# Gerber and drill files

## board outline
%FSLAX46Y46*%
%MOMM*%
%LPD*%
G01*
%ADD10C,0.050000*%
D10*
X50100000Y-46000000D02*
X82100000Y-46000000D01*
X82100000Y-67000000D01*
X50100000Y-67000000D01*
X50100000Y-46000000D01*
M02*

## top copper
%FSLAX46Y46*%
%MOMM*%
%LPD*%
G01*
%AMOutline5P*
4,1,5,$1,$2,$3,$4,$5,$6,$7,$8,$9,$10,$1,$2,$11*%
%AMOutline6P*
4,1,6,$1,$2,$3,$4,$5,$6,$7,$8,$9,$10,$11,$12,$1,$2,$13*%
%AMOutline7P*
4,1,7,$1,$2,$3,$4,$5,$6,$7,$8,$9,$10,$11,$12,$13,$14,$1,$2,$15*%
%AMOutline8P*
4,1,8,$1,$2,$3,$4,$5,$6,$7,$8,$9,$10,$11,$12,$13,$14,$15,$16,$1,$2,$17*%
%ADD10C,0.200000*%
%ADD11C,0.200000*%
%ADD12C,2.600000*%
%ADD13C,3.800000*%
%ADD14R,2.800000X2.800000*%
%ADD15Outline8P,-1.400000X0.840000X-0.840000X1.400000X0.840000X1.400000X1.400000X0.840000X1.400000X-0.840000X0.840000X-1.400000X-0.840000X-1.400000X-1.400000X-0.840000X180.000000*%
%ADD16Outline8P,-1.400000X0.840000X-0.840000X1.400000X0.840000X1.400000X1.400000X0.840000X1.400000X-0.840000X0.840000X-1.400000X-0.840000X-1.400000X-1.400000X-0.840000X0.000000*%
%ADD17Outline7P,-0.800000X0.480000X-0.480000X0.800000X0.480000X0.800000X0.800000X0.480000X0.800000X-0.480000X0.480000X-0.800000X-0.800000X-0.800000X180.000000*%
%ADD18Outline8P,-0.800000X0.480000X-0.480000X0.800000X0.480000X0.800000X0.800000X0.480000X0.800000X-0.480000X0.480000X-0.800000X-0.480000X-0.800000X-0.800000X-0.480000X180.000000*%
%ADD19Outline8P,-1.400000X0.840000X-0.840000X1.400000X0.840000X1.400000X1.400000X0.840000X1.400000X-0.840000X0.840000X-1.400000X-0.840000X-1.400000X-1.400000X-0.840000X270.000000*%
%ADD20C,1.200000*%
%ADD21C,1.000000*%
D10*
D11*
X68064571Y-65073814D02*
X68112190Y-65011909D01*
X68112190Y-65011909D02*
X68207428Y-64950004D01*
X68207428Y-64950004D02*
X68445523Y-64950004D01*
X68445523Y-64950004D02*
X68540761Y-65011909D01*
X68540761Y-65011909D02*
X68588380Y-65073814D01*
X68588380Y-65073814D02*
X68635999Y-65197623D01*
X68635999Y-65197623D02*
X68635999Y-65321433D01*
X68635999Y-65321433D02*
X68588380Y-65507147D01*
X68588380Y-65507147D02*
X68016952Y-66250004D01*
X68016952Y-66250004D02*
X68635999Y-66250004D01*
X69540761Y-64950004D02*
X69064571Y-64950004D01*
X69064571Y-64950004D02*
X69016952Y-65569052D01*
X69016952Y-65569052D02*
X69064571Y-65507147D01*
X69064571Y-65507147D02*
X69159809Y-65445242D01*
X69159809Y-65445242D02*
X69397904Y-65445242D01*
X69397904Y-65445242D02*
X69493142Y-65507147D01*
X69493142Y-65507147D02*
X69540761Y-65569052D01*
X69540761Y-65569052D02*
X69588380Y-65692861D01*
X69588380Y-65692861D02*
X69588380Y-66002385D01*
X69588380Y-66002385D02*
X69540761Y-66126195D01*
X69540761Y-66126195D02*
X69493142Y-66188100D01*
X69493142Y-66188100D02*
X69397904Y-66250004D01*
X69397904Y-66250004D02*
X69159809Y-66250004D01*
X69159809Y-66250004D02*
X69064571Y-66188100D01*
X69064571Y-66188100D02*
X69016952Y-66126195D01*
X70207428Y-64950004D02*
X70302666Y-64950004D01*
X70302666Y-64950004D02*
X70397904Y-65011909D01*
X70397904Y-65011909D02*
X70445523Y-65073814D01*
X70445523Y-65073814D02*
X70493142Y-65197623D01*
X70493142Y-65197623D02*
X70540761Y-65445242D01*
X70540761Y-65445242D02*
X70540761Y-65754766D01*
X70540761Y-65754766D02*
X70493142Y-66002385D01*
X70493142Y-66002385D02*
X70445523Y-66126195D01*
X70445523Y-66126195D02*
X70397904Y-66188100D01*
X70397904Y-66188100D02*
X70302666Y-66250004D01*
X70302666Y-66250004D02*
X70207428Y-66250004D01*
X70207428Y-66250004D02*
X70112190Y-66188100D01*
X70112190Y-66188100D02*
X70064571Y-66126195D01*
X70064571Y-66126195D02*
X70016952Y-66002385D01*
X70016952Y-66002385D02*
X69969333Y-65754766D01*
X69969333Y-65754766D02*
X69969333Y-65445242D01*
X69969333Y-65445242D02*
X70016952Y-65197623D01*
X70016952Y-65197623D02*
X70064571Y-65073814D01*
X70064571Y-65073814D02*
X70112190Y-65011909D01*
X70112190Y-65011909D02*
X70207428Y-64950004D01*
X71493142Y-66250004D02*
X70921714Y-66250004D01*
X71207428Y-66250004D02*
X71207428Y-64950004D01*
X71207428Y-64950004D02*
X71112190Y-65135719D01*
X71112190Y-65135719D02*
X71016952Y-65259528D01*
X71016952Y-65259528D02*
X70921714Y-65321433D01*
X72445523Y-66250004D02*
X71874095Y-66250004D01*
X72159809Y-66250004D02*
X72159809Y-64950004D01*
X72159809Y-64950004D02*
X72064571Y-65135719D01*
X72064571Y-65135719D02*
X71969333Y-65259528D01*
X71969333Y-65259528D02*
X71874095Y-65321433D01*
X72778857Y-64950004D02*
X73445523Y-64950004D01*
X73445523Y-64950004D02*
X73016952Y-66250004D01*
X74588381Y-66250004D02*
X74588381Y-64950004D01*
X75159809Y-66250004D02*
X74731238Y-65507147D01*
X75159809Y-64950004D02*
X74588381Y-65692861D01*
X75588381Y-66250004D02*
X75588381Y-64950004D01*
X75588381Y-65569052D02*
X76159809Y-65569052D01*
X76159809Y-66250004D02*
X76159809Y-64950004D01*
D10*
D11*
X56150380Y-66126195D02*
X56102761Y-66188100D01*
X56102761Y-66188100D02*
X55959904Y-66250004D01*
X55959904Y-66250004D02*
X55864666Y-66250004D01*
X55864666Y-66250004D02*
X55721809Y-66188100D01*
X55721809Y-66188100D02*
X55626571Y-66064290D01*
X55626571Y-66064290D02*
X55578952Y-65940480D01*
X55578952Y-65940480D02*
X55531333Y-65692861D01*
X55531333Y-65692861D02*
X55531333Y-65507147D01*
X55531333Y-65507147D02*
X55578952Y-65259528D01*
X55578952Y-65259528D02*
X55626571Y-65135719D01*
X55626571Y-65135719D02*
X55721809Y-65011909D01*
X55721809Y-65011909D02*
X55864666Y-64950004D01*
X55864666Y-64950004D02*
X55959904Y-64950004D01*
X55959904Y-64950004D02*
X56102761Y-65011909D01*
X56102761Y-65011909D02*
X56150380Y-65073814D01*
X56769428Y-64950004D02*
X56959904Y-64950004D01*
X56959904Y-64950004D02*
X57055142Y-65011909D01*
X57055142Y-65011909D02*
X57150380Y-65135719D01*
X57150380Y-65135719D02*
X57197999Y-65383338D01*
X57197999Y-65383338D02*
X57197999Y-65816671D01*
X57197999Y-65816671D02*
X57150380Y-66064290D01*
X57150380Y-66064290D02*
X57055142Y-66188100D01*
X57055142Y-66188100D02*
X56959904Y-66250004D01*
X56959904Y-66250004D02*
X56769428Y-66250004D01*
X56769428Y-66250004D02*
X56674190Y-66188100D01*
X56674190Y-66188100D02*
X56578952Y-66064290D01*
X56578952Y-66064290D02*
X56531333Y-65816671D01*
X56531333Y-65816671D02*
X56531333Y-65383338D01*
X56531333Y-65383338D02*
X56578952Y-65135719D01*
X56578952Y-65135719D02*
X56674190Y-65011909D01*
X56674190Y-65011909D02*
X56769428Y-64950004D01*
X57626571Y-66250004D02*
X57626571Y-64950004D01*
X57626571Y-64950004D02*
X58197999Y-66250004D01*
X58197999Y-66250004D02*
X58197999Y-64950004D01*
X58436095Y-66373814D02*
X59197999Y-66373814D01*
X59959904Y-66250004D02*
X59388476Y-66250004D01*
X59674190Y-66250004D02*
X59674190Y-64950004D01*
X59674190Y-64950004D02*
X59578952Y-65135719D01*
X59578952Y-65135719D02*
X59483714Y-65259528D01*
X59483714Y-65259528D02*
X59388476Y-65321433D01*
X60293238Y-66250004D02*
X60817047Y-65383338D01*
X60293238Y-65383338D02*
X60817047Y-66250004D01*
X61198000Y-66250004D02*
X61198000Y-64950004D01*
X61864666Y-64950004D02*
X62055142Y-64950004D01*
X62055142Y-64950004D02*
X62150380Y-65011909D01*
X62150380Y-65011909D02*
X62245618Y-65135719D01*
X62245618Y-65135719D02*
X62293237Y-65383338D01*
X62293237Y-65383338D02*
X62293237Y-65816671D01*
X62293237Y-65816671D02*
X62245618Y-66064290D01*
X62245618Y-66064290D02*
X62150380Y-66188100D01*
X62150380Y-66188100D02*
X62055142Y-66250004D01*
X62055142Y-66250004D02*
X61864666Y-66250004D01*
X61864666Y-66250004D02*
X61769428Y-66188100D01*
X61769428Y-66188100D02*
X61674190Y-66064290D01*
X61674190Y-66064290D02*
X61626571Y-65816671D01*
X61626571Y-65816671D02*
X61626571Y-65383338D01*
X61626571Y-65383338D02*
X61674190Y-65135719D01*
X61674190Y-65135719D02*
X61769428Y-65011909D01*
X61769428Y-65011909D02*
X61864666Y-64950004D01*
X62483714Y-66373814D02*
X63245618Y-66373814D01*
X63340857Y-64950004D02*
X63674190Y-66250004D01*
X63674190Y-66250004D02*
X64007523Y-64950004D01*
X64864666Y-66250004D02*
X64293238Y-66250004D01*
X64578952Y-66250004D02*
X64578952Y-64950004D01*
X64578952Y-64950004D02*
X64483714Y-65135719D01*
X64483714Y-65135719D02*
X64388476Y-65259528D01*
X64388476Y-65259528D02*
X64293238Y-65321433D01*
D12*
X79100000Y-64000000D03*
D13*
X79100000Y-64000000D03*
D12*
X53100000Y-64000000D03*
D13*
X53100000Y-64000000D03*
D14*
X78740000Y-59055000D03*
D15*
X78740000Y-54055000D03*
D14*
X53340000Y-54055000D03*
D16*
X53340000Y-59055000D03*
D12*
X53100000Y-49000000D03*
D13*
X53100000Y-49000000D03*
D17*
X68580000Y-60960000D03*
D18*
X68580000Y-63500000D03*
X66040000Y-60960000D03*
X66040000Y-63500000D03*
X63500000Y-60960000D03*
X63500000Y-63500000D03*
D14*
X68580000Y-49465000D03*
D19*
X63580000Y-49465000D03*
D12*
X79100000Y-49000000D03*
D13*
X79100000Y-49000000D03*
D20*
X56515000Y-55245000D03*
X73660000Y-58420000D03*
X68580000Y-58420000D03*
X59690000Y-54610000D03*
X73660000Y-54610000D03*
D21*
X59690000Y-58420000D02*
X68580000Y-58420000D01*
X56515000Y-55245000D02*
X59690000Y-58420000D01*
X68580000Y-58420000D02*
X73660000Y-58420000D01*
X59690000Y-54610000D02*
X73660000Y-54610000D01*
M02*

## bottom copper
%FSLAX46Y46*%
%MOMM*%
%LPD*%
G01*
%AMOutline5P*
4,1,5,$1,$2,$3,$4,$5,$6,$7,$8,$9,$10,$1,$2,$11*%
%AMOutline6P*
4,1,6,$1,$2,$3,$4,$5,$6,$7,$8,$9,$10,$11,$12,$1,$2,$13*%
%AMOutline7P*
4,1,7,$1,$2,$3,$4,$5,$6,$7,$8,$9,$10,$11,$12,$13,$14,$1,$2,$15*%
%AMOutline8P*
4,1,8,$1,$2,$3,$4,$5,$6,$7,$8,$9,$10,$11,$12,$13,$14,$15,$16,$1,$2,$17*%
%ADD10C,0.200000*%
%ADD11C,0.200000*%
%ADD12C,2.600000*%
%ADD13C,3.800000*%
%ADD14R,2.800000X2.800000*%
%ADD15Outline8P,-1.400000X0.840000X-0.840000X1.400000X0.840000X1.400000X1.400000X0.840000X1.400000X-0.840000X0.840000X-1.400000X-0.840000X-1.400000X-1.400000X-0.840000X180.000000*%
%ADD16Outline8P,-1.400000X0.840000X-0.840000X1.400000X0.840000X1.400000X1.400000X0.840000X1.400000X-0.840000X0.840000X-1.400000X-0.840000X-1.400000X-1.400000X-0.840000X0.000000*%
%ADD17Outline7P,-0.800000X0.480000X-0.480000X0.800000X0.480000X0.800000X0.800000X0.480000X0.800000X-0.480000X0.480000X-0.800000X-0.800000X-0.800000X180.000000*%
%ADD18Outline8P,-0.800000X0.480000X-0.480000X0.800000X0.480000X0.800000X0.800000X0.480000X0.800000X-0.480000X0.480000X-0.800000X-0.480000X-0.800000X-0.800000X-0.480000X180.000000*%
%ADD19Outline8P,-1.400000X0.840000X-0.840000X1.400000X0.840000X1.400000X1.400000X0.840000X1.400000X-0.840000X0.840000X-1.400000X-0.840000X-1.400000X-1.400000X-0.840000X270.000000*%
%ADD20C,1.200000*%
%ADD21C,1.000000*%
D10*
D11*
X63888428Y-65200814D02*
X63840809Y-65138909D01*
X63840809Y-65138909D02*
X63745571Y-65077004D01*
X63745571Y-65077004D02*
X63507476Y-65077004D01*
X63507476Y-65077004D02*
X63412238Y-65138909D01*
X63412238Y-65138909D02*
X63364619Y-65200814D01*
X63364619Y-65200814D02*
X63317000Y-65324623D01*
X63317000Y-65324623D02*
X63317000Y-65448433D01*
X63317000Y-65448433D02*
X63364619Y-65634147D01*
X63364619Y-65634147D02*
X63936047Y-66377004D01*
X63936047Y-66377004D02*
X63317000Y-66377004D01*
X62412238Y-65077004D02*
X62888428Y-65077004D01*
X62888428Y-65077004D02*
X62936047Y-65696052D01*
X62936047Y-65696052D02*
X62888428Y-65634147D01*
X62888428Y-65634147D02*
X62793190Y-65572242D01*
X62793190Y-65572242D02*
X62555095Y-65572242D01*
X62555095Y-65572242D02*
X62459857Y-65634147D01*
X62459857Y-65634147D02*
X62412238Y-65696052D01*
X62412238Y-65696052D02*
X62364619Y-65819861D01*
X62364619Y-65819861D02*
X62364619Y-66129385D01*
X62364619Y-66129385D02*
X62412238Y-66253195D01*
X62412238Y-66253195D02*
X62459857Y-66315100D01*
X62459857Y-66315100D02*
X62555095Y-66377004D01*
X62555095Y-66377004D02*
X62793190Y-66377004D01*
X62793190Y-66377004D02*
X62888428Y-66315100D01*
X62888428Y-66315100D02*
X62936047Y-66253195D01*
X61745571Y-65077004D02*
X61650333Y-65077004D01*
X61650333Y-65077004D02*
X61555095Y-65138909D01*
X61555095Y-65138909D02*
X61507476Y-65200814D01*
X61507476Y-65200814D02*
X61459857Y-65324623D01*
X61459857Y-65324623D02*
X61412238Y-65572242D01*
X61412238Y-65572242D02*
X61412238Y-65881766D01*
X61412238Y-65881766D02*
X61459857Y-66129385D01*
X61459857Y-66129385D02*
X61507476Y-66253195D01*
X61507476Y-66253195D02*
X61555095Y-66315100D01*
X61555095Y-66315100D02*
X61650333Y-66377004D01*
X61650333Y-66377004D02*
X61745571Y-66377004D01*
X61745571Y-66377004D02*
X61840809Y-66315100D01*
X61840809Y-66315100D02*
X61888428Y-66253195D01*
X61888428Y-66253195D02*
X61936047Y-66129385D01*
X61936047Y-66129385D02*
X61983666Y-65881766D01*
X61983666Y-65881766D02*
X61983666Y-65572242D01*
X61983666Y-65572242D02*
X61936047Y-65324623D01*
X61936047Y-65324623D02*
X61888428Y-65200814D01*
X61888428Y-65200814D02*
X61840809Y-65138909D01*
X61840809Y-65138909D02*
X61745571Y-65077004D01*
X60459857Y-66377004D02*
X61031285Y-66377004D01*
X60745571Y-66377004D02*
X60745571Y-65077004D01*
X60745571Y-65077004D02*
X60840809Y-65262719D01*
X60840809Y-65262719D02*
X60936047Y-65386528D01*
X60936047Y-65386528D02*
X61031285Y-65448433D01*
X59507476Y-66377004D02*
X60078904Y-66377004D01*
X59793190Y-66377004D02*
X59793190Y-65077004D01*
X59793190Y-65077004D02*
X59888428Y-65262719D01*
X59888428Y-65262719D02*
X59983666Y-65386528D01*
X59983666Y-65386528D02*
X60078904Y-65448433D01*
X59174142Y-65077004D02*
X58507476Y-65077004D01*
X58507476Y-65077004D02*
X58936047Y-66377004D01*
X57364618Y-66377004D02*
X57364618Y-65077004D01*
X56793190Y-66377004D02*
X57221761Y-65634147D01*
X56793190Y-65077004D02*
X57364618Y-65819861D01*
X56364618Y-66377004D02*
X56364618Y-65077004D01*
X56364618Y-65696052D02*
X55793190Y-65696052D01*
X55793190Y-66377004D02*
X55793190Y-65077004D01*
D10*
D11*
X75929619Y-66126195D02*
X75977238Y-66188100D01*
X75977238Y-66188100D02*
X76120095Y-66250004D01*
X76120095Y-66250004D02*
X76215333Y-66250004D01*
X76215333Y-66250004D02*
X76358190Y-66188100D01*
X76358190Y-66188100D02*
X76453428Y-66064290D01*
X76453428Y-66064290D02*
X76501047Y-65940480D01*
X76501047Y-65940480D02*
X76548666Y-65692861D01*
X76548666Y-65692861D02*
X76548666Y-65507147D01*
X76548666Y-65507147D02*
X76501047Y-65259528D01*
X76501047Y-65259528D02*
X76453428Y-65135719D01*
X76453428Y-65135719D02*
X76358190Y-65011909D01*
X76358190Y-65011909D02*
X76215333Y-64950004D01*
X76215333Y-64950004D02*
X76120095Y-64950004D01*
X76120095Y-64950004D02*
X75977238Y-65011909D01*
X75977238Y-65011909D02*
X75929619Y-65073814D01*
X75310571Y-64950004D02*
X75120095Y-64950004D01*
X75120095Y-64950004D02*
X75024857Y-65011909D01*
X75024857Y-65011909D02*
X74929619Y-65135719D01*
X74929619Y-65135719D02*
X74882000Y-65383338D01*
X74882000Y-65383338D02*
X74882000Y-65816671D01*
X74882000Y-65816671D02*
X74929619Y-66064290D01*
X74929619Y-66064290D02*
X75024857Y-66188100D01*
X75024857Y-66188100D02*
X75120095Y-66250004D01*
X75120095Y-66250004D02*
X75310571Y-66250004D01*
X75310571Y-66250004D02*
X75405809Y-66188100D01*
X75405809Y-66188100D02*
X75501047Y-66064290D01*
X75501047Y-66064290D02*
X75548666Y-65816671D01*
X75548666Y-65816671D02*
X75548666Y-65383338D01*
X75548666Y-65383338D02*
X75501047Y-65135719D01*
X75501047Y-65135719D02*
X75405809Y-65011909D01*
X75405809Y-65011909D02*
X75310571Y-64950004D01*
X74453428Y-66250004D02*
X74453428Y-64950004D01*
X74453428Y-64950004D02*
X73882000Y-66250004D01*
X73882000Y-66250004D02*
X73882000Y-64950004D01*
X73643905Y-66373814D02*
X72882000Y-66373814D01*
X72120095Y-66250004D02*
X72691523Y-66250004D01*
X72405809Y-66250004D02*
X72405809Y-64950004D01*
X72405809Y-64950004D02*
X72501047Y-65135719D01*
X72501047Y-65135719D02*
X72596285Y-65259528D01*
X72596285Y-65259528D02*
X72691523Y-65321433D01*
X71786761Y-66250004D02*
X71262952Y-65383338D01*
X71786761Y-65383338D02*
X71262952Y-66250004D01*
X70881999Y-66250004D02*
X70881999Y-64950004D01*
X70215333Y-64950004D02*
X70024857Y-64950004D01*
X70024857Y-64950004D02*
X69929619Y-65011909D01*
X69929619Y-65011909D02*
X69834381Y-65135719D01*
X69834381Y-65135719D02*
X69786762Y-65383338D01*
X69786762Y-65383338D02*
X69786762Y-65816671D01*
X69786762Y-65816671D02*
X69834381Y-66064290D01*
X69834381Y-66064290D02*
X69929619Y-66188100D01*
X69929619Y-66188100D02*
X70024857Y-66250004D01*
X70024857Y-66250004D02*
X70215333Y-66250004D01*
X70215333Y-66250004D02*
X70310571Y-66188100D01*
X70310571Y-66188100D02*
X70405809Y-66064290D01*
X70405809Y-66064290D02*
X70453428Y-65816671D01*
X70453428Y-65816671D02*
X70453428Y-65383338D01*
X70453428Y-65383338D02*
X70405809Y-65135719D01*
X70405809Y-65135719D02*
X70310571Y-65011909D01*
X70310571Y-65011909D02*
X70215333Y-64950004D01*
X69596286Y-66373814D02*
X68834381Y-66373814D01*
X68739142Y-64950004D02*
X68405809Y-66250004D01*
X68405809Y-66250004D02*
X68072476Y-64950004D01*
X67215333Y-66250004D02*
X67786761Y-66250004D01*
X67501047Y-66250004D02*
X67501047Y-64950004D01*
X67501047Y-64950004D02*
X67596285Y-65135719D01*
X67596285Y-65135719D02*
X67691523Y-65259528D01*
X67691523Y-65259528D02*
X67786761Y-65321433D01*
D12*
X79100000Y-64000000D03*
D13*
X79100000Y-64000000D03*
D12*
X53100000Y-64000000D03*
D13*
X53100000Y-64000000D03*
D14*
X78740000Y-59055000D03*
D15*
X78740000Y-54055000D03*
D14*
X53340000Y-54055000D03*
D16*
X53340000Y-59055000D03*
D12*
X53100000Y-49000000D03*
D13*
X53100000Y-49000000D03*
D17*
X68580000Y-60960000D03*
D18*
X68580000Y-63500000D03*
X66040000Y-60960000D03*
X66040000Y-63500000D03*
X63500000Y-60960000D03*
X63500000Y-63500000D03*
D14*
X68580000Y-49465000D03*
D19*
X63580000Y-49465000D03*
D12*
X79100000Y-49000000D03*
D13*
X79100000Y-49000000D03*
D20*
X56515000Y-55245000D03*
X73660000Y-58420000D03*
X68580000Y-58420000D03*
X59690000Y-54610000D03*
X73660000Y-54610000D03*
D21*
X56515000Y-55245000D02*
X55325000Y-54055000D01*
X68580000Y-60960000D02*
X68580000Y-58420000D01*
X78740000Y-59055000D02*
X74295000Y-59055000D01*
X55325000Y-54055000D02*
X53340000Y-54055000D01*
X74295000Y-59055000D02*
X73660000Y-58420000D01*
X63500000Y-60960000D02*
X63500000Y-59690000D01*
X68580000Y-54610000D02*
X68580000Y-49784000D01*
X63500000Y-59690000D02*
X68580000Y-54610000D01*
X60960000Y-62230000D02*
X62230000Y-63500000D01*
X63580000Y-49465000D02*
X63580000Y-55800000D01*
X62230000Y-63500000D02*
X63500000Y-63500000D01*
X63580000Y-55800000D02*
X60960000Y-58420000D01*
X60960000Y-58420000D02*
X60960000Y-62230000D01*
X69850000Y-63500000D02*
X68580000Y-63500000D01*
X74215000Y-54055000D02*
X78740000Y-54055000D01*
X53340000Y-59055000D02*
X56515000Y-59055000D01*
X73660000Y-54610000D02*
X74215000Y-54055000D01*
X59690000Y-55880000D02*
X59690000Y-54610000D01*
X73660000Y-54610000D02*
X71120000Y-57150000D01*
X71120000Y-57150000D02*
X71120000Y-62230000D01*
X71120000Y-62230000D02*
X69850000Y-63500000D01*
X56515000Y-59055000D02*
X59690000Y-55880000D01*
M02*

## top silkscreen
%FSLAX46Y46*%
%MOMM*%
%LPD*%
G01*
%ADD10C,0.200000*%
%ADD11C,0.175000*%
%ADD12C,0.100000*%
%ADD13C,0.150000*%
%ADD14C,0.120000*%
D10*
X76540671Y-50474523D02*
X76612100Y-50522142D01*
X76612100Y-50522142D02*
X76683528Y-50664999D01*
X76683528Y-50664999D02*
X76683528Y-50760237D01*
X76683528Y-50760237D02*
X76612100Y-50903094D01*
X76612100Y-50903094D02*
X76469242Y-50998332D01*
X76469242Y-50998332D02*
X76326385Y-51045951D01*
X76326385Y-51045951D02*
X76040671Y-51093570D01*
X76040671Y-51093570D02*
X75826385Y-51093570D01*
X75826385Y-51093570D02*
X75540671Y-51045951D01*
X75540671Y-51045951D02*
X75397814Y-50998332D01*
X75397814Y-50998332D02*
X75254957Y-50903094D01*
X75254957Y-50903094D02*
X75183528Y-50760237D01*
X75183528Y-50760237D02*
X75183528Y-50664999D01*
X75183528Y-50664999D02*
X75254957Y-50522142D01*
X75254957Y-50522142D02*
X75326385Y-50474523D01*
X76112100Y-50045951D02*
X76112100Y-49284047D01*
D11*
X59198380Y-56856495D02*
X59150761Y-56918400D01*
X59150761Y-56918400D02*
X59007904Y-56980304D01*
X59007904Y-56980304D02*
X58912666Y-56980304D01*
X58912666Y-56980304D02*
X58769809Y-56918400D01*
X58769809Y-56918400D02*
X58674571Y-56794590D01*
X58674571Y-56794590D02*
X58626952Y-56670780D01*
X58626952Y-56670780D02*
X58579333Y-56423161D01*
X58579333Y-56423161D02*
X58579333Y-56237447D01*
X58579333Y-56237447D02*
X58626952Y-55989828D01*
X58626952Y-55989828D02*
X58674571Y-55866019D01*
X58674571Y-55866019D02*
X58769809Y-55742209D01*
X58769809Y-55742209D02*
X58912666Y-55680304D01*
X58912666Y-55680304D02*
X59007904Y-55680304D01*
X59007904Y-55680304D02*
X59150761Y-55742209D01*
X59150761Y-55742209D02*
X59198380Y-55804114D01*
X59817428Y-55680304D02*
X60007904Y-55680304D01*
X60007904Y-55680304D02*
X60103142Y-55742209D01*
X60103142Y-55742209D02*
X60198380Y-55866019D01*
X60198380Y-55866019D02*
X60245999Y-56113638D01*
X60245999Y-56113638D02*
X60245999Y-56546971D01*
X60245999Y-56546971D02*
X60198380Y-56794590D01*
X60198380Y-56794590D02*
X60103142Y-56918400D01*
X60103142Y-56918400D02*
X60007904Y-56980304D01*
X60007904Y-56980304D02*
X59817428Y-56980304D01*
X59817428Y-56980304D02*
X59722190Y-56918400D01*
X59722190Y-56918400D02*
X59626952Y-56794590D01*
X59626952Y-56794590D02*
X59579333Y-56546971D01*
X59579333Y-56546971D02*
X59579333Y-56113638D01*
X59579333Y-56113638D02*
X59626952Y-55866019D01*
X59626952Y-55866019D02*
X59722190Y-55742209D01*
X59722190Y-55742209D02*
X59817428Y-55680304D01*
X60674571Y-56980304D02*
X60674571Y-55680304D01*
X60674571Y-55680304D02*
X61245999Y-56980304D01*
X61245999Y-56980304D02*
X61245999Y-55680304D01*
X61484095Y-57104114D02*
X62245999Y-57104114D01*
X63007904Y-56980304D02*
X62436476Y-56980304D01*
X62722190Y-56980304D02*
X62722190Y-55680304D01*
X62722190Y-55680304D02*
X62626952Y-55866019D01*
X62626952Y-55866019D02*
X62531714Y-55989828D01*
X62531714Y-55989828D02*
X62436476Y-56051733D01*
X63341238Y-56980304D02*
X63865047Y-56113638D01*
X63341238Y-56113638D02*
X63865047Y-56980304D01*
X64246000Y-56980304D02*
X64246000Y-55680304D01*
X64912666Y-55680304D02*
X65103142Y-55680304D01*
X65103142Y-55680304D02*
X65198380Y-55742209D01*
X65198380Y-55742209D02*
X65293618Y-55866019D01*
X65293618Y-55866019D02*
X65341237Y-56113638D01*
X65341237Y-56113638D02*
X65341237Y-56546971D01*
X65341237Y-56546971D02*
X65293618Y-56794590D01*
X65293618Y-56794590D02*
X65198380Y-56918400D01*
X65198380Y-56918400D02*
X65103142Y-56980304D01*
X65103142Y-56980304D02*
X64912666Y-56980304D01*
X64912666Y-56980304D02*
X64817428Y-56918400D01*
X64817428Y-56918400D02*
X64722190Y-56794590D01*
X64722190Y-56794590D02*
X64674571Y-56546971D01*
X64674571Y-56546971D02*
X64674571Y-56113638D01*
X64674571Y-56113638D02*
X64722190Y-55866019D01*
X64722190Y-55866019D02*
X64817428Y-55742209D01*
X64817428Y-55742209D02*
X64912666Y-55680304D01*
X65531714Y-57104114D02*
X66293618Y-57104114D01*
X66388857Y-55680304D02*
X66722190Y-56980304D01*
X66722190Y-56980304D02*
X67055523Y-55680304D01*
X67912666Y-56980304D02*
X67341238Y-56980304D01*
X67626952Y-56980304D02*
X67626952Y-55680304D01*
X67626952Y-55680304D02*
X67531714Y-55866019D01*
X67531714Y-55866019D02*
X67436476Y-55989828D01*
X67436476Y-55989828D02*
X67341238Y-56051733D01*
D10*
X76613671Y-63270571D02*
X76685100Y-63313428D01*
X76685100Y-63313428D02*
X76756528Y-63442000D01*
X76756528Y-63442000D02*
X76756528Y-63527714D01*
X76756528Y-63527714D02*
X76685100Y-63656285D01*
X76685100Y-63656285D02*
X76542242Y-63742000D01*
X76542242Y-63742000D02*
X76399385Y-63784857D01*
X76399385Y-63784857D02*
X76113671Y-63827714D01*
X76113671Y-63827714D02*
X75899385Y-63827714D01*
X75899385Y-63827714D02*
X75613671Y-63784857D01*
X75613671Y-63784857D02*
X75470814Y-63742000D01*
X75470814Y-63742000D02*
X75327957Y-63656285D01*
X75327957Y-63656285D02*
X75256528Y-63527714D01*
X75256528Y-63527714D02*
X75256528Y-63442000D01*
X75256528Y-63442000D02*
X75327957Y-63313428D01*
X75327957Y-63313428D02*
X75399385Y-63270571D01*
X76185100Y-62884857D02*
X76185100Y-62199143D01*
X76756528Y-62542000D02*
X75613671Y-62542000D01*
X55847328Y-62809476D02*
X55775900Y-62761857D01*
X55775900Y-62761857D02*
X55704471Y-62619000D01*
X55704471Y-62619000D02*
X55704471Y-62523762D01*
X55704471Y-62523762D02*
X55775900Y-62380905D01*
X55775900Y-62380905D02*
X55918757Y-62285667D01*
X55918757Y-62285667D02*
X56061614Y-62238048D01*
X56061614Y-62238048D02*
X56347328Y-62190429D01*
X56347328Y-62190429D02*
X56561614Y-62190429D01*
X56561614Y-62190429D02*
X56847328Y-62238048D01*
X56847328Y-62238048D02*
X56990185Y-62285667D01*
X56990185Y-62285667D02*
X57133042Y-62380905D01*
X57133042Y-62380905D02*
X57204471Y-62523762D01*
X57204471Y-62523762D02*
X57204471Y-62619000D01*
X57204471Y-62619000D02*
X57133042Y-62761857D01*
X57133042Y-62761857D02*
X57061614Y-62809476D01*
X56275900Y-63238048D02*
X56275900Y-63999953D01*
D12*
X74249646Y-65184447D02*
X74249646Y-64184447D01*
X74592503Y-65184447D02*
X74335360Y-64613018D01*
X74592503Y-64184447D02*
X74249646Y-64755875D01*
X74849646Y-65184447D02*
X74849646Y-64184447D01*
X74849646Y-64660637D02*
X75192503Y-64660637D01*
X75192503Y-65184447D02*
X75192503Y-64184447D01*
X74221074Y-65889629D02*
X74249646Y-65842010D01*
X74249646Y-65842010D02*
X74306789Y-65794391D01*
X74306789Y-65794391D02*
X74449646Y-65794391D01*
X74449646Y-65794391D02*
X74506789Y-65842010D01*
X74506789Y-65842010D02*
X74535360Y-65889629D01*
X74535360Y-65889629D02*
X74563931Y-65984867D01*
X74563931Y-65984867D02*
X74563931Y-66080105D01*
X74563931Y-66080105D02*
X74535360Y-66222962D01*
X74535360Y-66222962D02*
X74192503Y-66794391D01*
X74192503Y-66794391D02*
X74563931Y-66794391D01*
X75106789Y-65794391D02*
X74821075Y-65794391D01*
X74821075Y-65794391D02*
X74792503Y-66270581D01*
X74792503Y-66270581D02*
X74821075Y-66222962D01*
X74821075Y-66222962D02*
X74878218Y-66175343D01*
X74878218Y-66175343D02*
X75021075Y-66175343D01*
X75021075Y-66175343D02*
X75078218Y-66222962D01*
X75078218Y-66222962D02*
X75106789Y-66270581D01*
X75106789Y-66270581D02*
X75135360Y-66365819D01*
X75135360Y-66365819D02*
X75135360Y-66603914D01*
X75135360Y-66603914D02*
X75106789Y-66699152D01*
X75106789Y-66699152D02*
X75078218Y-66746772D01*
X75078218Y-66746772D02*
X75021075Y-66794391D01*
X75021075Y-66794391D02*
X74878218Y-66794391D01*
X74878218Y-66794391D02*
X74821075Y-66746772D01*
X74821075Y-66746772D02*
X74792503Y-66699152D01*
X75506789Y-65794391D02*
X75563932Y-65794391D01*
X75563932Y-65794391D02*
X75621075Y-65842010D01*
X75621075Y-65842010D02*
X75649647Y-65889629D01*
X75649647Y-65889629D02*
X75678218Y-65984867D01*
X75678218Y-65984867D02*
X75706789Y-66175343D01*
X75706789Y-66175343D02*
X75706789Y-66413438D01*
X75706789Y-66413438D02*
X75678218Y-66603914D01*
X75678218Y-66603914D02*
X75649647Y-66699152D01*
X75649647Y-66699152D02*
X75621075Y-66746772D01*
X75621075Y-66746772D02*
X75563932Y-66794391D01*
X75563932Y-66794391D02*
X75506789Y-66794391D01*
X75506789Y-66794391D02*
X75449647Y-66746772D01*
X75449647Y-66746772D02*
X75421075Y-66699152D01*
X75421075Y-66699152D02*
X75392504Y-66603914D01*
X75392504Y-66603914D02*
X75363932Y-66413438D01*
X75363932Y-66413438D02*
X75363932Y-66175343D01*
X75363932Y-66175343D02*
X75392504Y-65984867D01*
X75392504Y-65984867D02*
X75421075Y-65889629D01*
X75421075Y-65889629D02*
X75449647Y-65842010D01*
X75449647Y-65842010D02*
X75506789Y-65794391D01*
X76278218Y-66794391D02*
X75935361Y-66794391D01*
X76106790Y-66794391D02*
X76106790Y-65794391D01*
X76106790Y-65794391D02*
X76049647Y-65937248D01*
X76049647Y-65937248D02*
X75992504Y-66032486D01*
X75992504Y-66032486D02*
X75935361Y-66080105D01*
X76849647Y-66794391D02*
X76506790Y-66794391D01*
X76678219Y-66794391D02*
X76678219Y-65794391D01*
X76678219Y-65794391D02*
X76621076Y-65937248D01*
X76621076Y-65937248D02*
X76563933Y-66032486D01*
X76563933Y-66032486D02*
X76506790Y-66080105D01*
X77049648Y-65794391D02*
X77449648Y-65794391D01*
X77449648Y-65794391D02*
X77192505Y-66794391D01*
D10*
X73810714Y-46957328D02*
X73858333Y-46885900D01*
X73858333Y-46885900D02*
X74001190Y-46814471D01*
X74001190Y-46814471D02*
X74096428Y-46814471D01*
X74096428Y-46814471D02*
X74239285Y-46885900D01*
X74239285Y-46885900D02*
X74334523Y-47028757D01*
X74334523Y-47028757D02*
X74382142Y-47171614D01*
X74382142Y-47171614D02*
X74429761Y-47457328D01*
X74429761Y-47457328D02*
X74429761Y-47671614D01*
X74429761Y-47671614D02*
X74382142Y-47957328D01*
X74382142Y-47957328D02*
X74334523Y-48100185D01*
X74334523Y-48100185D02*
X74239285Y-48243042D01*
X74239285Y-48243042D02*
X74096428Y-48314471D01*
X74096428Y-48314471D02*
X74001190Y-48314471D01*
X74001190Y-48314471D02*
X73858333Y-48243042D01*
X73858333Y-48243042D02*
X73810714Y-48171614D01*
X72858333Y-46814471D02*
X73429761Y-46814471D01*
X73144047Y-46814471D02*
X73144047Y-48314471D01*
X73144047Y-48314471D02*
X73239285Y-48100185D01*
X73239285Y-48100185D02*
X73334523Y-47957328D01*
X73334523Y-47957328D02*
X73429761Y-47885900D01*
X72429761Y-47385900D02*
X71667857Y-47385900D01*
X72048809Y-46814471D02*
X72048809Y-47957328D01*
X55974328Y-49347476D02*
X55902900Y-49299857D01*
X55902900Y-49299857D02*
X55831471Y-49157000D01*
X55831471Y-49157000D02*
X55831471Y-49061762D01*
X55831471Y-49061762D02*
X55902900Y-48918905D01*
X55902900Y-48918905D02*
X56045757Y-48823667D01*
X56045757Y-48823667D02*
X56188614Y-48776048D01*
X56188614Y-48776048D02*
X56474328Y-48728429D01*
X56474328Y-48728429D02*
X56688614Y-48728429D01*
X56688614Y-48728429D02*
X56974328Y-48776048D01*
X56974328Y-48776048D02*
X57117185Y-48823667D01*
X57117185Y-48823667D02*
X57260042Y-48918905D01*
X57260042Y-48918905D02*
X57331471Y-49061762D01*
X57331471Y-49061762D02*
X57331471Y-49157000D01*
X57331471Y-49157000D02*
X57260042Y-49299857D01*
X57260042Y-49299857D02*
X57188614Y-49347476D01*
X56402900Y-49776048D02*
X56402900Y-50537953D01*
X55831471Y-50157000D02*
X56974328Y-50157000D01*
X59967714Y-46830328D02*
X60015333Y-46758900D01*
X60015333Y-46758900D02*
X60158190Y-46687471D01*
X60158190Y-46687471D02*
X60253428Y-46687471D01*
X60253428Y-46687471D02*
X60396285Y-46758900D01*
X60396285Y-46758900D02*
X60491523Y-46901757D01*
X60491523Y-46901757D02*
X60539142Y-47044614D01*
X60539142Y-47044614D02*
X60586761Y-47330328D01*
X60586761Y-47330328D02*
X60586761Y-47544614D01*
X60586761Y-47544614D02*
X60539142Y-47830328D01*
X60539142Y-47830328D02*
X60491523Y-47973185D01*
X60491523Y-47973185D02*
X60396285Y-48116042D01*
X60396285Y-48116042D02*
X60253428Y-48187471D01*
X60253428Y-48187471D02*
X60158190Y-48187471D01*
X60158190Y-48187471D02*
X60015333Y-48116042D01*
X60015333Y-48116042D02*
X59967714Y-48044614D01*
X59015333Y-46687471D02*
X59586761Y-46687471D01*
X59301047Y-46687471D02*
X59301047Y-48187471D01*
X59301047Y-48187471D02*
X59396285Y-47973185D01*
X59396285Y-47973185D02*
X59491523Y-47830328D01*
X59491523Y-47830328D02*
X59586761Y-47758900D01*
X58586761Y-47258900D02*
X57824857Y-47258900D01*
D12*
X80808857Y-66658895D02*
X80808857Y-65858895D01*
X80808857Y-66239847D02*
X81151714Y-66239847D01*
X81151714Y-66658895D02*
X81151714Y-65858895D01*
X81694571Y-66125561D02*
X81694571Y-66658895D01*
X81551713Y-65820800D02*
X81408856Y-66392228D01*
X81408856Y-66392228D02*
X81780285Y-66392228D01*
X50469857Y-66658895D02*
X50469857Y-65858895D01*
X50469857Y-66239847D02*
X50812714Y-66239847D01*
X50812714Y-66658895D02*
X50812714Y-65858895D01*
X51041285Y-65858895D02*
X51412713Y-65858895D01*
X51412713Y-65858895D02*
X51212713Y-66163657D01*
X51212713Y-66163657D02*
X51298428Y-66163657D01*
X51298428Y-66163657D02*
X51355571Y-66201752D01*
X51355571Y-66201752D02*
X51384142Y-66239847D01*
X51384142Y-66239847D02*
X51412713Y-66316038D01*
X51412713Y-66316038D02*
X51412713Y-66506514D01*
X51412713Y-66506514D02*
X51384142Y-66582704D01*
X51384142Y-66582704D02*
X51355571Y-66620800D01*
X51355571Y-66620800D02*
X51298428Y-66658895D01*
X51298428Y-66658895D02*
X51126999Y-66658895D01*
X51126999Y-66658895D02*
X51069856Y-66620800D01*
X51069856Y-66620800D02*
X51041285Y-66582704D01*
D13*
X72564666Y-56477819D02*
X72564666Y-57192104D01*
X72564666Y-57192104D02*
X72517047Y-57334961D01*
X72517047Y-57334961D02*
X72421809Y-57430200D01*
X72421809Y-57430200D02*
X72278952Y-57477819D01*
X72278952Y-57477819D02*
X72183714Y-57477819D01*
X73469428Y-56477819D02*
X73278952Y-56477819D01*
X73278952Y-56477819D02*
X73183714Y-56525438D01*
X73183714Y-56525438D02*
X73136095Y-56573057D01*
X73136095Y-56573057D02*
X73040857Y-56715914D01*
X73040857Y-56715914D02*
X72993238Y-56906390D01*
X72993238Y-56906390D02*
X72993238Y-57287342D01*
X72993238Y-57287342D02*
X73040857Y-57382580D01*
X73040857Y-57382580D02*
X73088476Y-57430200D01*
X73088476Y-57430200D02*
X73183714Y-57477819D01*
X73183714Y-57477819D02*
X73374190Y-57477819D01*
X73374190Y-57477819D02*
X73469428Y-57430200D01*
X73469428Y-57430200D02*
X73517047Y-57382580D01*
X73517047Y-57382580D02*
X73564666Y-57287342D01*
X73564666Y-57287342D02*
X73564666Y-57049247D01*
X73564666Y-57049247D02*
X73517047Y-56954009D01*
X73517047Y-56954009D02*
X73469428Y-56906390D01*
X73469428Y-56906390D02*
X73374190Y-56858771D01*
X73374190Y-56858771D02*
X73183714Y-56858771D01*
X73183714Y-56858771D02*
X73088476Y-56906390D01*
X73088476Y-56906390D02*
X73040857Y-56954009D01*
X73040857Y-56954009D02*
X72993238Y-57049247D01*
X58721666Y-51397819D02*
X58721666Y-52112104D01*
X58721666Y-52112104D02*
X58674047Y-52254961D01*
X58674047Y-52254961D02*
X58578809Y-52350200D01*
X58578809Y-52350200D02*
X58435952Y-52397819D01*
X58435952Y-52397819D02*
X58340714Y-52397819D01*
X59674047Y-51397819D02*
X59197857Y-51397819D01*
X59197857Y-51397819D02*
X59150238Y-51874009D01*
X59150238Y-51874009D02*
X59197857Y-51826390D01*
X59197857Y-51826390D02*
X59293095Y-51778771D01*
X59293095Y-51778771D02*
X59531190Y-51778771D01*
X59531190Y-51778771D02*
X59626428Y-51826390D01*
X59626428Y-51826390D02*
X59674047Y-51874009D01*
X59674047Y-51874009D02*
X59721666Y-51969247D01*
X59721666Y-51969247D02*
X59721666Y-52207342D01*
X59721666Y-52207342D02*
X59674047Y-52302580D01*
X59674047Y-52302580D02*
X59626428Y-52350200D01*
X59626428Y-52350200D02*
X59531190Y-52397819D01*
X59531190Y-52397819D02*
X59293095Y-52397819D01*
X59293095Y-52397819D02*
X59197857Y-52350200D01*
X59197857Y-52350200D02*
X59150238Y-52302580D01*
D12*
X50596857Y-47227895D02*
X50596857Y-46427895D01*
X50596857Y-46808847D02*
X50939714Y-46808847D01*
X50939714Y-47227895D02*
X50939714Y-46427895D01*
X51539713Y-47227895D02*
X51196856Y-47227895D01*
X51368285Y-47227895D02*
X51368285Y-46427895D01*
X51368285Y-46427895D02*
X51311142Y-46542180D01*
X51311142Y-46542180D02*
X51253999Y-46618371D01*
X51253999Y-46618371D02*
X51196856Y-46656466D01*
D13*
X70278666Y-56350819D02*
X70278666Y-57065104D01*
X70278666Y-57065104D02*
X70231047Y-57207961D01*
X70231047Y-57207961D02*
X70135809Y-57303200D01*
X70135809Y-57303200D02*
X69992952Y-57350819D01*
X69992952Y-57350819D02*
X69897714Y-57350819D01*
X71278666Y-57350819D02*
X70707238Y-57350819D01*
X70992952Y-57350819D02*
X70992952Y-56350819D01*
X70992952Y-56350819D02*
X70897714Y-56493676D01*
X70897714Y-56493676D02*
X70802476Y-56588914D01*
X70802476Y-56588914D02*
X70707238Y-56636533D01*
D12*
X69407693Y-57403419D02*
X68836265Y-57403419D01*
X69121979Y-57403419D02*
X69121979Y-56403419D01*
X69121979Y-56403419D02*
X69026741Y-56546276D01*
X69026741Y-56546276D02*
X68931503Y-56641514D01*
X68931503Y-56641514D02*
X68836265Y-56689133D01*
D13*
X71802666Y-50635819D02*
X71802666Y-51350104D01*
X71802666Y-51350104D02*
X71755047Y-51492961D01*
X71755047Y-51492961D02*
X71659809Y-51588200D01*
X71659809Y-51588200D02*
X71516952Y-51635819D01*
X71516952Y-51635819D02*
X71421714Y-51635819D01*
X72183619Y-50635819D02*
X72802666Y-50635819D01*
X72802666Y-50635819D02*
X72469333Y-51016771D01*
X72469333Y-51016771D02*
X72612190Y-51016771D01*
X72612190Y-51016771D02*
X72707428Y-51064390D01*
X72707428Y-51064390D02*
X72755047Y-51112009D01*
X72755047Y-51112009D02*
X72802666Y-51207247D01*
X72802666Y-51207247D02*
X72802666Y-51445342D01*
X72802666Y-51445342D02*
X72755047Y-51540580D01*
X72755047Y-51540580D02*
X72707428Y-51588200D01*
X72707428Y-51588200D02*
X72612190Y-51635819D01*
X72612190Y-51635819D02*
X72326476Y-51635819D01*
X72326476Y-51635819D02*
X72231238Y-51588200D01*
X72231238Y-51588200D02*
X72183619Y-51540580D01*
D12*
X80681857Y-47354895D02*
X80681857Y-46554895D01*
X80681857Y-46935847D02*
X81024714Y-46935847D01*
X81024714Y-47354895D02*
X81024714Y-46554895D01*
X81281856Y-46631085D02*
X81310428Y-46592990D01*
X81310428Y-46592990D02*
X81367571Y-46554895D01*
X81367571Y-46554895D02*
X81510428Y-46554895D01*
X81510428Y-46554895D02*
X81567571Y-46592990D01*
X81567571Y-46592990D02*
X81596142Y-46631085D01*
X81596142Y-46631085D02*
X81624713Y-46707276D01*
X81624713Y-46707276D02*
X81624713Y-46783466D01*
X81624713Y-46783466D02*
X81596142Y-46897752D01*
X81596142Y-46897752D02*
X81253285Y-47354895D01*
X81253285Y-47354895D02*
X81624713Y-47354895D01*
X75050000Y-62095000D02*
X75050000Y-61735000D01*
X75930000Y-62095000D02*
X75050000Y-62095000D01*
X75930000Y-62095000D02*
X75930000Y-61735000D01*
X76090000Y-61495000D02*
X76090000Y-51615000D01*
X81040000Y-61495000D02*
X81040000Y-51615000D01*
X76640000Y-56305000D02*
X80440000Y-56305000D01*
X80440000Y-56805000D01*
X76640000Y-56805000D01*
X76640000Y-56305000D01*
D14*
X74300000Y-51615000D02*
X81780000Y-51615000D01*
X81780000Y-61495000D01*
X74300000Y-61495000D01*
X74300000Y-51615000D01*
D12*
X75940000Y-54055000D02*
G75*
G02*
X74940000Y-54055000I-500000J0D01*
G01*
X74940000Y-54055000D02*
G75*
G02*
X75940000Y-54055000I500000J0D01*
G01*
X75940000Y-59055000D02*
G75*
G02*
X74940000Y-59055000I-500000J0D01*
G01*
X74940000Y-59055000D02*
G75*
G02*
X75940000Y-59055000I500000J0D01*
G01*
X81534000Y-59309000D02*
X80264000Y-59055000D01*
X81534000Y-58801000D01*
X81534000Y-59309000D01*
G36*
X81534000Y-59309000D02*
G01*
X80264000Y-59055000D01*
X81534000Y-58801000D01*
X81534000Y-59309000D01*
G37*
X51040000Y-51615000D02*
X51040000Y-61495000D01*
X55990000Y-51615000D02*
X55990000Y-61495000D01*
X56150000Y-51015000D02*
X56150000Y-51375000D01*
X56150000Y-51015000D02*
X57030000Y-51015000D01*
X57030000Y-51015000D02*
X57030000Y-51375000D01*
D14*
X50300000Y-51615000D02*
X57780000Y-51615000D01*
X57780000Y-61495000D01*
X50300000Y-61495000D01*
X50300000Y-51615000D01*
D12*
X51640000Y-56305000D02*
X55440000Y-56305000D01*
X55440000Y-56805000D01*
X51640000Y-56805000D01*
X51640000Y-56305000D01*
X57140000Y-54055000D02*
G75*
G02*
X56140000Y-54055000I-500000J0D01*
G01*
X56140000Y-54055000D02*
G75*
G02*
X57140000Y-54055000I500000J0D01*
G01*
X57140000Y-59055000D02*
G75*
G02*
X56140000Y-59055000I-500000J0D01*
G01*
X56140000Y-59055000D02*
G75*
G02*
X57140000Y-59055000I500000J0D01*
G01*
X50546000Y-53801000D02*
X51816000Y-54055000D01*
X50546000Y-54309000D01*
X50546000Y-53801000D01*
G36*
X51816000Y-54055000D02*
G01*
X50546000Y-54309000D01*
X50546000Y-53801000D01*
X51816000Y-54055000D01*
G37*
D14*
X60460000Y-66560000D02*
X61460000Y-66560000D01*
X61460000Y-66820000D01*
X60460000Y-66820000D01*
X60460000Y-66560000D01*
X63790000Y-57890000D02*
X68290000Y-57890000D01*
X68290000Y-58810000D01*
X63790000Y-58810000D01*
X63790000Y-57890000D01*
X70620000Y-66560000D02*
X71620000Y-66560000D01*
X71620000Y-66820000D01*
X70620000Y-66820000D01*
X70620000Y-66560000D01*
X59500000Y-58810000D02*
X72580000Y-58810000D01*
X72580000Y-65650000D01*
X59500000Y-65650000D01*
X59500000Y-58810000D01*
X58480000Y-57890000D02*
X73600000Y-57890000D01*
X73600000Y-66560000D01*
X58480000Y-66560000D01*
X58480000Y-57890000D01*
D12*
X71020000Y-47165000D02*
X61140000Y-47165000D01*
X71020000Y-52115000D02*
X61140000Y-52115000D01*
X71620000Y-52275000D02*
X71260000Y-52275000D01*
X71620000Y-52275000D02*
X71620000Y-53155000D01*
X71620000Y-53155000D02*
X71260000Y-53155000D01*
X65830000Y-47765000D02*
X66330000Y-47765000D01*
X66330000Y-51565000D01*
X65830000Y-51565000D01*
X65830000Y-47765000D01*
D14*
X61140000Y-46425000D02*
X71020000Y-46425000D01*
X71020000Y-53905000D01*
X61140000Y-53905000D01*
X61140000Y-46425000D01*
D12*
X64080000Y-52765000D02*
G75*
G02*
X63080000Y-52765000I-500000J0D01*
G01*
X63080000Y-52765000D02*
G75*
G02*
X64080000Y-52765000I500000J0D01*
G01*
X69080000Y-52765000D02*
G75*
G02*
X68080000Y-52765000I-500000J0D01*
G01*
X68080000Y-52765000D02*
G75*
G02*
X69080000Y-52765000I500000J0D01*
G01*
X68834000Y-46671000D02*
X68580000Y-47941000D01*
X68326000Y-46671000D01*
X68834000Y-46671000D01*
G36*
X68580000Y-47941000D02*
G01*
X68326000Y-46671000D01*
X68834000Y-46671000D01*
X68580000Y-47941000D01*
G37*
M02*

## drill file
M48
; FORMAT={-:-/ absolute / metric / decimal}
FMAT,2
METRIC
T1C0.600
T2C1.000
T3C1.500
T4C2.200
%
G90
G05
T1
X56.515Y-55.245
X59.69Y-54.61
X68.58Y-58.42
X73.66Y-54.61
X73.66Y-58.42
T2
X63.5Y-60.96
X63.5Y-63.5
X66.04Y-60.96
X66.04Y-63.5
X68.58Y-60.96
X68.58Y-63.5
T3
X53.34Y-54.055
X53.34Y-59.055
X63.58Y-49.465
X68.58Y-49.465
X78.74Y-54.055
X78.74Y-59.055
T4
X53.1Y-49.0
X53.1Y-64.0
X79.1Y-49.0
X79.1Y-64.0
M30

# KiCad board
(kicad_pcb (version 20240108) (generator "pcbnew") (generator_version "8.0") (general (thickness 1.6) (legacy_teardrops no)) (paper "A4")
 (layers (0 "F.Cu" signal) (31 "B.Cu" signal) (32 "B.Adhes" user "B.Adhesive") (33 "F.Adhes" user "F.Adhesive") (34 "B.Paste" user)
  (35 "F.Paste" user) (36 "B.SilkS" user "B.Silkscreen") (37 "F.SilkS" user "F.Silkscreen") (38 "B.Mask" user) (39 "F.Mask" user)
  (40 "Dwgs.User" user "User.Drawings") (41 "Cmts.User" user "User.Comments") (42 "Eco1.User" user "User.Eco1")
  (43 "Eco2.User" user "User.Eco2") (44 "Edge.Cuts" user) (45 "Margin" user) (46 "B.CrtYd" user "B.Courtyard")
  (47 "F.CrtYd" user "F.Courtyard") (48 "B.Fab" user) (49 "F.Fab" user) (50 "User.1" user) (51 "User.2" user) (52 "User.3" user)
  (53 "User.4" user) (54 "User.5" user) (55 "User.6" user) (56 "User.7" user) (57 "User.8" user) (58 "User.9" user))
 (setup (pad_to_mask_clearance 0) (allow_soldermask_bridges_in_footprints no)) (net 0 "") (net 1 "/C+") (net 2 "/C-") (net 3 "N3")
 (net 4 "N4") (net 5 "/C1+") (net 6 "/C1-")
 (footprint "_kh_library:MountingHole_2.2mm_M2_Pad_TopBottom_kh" (layer "F.Cu") (at 79.1 64)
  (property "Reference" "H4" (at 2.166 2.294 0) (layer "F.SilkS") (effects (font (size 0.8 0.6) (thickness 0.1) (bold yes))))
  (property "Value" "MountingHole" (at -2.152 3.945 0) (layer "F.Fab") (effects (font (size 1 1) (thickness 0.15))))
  (pad "1" thru_hole circle (at 0 0) (size 2.6 2.6) (drill 2.2) (layers "*.Cu" "*.Mask") (remove_unused_layers no))
  (pad "1" connect circle (at 0 0) (size 3.8 3.8) (layers "F.Cu" "F.Mask"))
  (pad "1" connect circle (at 0 0) (size 3.8 3.8) (layers "B.Cu" "B.Mask")))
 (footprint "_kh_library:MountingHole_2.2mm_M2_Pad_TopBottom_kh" (layer "F.Cu") (at 53.1 64)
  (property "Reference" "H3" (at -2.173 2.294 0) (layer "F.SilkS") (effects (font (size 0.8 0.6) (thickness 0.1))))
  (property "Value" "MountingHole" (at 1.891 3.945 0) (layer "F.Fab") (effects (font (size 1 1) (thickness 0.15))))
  (pad "1" thru_hole circle (at 0 0) (size 2.6 2.6) (drill 2.2) (layers "*.Cu" "*.Mask") (remove_unused_layers no))
  (pad "1" connect circle (at 0 0) (size 3.8 3.8) (layers "F.Cu" "F.Mask"))
  (pad "1" connect circle (at 0 0) (size 3.8 3.8) (layers "B.Cu" "B.Mask")))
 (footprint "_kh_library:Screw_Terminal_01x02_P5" (layer "F.Cu") (at 78.74 59.055 180)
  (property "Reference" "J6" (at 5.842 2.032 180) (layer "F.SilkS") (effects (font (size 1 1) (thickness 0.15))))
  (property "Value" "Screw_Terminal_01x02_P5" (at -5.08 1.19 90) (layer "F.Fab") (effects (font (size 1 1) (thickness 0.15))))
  (fp_line (start 3.69 -3.04) (end 3.69 -2.68) (stroke (width 0.1) (type default)) (layer "F.SilkS"))
  (fp_line (start 2.81 -3.04) (end 3.69 -3.04) (stroke (width 0.1) (type default)) (layer "F.SilkS"))
  (fp_line (start 2.81 -3.04) (end 2.81 -2.68) (stroke (width 0.1) (type default)) (layer "F.SilkS"))
  (fp_line (start 2.65 -2.44) (end 2.65 7.44) (stroke (width 0.1) (type default)) (layer "F.SilkS"))
  (fp_line (start -2.3 -2.44) (end -2.3 7.44) (stroke (width 0.1) (type default)) (layer "F.SilkS"))
  (fp_rect (start -1.7 2.25) (end 2.1 2.75) (stroke (width 0.1) (type default)) (fill none) (layer "F.SilkS"))
  (fp_rect (start -3.04 -2.44) (end 4.44 7.44) (stroke (width 0.12) (type default)) (fill none) (layer "F.SilkS"))
  (fp_circle (center 3.3 5) (end 3.8 5) (stroke (width 0.1) (type default)) (fill none) (layer "F.SilkS"))
  (fp_circle (center 3.3 0) (end 3.8 0) (stroke (width 0.1) (type default)) (fill none) (layer "F.SilkS"))
  (fp_poly (pts (xy -2.794 -0.254) (xy -1.524 0) (xy -2.794 0.254)) (stroke (width 0.1) (type solid)) (fill solid) (layer "F.SilkS"))
  (pad "1" thru_hole rect (at 0 0 180) (size 2.8 2.8) (drill 1.5) (layers "*.Cu" "*.Mask") (remove_unused_layers no) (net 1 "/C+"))
  (pad "2" thru_hole roundrect (at 0 5 180) (size 2.8 2.8) (drill 1.5) (layers "*.Cu" "*.Mask") (remove_unused_layers no)
   (roundrect_rratio 0) (chamfer_ratio 0.2) (chamfer top_left top_right bottom_left bottom_right) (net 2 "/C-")))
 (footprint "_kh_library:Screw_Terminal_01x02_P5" (layer "F.Cu") (at 53.34 54.055)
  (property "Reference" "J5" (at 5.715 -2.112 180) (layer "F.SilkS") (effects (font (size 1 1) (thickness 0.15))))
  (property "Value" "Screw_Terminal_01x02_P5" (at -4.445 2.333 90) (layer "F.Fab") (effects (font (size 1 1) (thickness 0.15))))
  (fp_line (start -2.3 -2.44) (end -2.3 7.44) (stroke (width 0.1) (type default)) (layer "F.SilkS"))
  (fp_line (start 2.65 -2.44) (end 2.65 7.44) (stroke (width 0.1) (type default)) (layer "F.SilkS"))
  (fp_line (start 2.81 -3.04) (end 2.81 -2.68) (stroke (width 0.1) (type default)) (layer "F.SilkS"))
  (fp_line (start 2.81 -3.04) (end 3.69 -3.04) (stroke (width 0.1) (type default)) (layer "F.SilkS"))
  (fp_line (start 3.69 -3.04) (end 3.69 -2.68) (stroke (width 0.1) (type default)) (layer "F.SilkS"))
  (fp_rect (start -3.04 -2.44) (end 4.44 7.44) (stroke (width 0.12) (type default)) (fill none) (layer "F.SilkS"))
  (fp_rect (start -1.7 2.25) (end 2.1 2.75) (stroke (width 0.1) (type default)) (fill none) (layer "F.SilkS"))
  (fp_circle (center 3.3 0) (end 3.8 0) (stroke (width 0.1) (type default)) (fill none) (layer "F.SilkS"))
  (fp_circle (center 3.3 5) (end 3.8 5) (stroke (width 0.1) (type default)) (fill none) (layer "F.SilkS"))
  (fp_poly (pts (xy -2.794 -0.254) (xy -1.524 0) (xy -2.794 0.254)) (stroke (width 0.1) (type solid)) (fill solid) (layer "F.SilkS"))
  (pad "1" thru_hole rect (at 0 0) (size 2.8 2.8) (drill 1.5) (layers "*.Cu" "*.Mask") (remove_unused_layers no) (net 1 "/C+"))
  (pad "2" thru_hole roundrect (at 0 5) (size 2.8 2.8) (drill 1.5) (layers "*.Cu" "*.Mask") (remove_unused_layers no) (roundrect_rratio 0)
   (chamfer_ratio 0.2) (chamfer top_left top_right bottom_left bottom_right) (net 2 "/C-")))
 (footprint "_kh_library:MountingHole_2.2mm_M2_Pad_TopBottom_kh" (layer "F.Cu") (at 53.1 49)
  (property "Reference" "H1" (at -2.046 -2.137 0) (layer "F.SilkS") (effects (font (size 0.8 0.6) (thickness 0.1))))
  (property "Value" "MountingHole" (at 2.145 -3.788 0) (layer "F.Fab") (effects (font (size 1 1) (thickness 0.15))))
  (pad "1" thru_hole circle (at 0 0) (size 2.6 2.6) (drill 2.2) (layers "*.Cu" "*.Mask") (remove_unused_layers no))
  (pad "1" connect circle (at 0 0) (size 3.8 3.8) (layers "F.Cu" "F.Mask"))
  (pad "1" connect circle (at 0 0) (size 3.8 3.8) (layers "B.Cu" "B.Mask")))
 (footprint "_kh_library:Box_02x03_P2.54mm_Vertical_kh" (layer "F.Cu") (at 68.58 60.96 180)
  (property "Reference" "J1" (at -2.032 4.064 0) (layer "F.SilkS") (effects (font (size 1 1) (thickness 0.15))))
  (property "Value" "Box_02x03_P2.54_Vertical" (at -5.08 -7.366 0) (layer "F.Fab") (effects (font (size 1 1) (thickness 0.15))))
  (fp_rect (start 7.12 -5.6) (end 8.12 -5.86) (stroke (width 0.12) (type default)) (fill none) (layer "F.SilkS"))
  (fp_rect (start 0.29 3.07) (end 4.79 2.15) (stroke (width 0.12) (type default)) (fill none) (layer "F.SilkS"))
  (fp_rect (start -3.04 -5.6) (end -2.04 -5.86) (stroke (width 0.12) (type default)) (fill none) (layer "F.SilkS"))
  (fp_rect (start -4 2.15) (end 9.08 -4.69) (stroke (width 0.12) (type default)) (fill none) (layer "F.SilkS"))
  (fp_rect (start -5.02 3.07) (end 10.1 -5.6) (stroke (width 0.12) (type default)) (fill none) (layer "F.SilkS"))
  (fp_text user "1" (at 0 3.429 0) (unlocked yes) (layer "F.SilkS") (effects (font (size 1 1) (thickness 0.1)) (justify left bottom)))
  (pad "1" thru_hole roundrect (at 0 0 180) (size 1.6 1.6) (drill 1) (layers "*.Cu" "*.Mask") (remove_unused_layers no) (roundrect_rratio 0)
   (chamfer_ratio 0.2) (chamfer top_left top_right bottom_right) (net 1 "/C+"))
  (pad "2" thru_hole roundrect (at 0 -2.54 180) (size 1.6 1.6) (drill 1) (layers "*.Cu" "*.Mask") (remove_unused_layers no)
   (roundrect_rratio 0) (chamfer_ratio 0.2) (chamfer top_left top_right bottom_left bottom_right) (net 2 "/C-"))
  (pad "3" thru_hole roundrect (at 2.54 0 180) (size 1.6 1.6) (drill 1) (layers "*.Cu" "*.Mask") (remove_unused_layers no)
   (roundrect_rratio 0) (chamfer_ratio 0.2) (chamfer top_left top_right bottom_left bottom_right) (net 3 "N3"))
  (pad "4" thru_hole roundrect (at 2.54 -2.54 180) (size 1.6 1.6) (drill 1) (layers "*.Cu" "*.Mask") (remove_unused_layers no)
   (roundrect_rratio 0) (chamfer_ratio 0.2) (chamfer top_left top_right bottom_left bottom_right) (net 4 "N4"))
  (pad "5" thru_hole roundrect (at 5.08 0 180) (size 1.6 1.6) (drill 1) (layers "*.Cu" "*.Mask") (remove_unused_layers no)
   (roundrect_rratio 0) (chamfer_ratio 0.2) (chamfer top_left top_right bottom_left bottom_right) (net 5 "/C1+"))
  (pad "6" thru_hole roundrect (at 5.08 -2.54 180) (size 1.6 1.6) (drill 1) (layers "*.Cu" "*.Mask") (remove_unused_layers no)
   (roundrect_rratio 0) (chamfer_ratio 0.2) (chamfer top_left top_right bottom_left bottom_right) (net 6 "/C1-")))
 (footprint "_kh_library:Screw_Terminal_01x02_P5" (layer "F.Cu") (at 68.58 49.465 -90)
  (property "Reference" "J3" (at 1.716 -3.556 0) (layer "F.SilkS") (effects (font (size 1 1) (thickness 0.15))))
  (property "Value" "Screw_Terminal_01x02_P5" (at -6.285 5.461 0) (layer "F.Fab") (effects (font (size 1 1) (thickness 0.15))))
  (fp_line (start -2.3 -2.44) (end -2.3 7.44) (stroke (width 0.1) (type default)) (layer "F.SilkS"))
  (fp_line (start 2.65 -2.44) (end 2.65 7.44) (stroke (width 0.1) (type default)) (layer "F.SilkS"))
  (fp_line (start 2.81 -3.04) (end 2.81 -2.68) (stroke (width 0.1) (type default)) (layer "F.SilkS"))
  (fp_line (start 2.81 -3.04) (end 3.69 -3.04) (stroke (width 0.1) (type default)) (layer "F.SilkS"))
  (fp_line (start 3.69 -3.04) (end 3.69 -2.68) (stroke (width 0.1) (type default)) (layer "F.SilkS"))
  (fp_rect (start -1.7 2.25) (end 2.1 2.75) (stroke (width 0.1) (type default)) (fill none) (layer "F.SilkS"))
  (fp_rect (start -3.04 -2.44) (end 4.44 7.44) (stroke (width 0.12) (type default)) (fill none) (layer "F.SilkS"))
  (fp_circle (center 3.3 5) (end 3.8 5) (stroke (width 0.1) (type default)) (fill none) (layer "F.SilkS"))
  (fp_circle (center 3.3 0) (end 3.8 0) (stroke (width 0.1) (type default)) (fill none) (layer "F.SilkS"))
  (fp_poly (pts (xy -2.794 -0.254) (xy -1.524 0) (xy -2.794 0.254)) (stroke (width 0.1) (type solid)) (fill solid) (layer "F.SilkS"))
  (pad "1" thru_hole rect (at 0 0 270) (size 2.8 2.8) (drill 1.5) (layers "*.Cu" "*.Mask") (remove_unused_layers no) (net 5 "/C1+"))
  (pad "2" thru_hole roundrect (at 0 5 270) (size 2.8 2.8) (drill 1.5) (layers "*.Cu" "*.Mask") (remove_unused_layers no)
   (roundrect_rratio 0) (chamfer_ratio 0.2) (chamfer top_left top_right bottom_left bottom_right) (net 6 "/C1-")))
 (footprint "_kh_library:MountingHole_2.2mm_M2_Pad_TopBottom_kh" (layer "F.Cu") (at 79.1 49)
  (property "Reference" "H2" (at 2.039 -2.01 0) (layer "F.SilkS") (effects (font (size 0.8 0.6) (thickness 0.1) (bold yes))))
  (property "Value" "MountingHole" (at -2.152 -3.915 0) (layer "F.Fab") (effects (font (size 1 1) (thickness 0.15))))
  (pad "1" thru_hole circle (at 0 0) (size 2.6 2.6) (drill 2.2) (layers "*.Cu" "*.Mask") (remove_unused_layers no))
  (pad "1" connect circle (at 0 0) (size 3.8 3.8) (layers "F.Cu" "F.Mask"))
  (pad "1" connect circle (at 0 0) (size 3.8 3.8) (layers "B.Cu" "B.Mask")))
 (gr_rect (start 50.1 46) (end 82.1 67) (stroke (width 0.05) (type default)) (fill none) (layer "Edge.Cuts"))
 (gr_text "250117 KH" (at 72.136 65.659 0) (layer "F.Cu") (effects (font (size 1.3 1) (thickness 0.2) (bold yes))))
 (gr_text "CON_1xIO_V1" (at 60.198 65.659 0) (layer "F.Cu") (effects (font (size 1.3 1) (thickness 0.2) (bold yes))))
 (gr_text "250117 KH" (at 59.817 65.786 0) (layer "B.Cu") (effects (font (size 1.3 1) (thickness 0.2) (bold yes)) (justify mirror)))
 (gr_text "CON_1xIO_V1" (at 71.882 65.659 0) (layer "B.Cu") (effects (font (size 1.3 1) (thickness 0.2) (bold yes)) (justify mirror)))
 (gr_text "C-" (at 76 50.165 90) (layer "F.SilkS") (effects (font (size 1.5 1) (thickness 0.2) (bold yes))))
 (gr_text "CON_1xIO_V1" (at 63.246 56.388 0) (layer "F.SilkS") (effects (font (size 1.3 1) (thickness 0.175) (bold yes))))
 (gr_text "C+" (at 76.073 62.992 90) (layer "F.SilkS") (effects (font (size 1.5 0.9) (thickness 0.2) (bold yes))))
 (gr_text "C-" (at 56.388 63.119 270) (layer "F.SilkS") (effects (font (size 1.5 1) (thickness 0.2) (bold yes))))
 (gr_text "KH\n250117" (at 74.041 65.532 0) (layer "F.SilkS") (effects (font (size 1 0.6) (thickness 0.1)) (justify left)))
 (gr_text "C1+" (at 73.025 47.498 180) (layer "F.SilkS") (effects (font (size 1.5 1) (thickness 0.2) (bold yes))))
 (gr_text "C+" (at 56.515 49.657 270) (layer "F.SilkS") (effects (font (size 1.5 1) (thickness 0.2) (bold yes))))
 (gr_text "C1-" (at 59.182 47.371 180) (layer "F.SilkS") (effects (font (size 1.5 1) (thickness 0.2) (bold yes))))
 (segment (start 59.69 58.42) (end 68.58 58.42) (width 1) (layer "F.Cu") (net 1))
 (segment (start 56.515 55.245) (end 59.69 58.42) (width 1) (layer "F.Cu") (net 1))
 (segment (start 68.58 58.42) (end 73.66 58.42) (width 1) (layer "F.Cu") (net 1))
 (via (at 56.515 55.245) (size 1.2) (drill 0.6) (layers "F.Cu" "B.Cu") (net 1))
 (via (at 73.66 58.42) (size 1.2) (drill 0.6) (layers "F.Cu" "B.Cu") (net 1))
 (via (at 68.58 58.42) (size 1.2) (drill 0.6) (layers "F.Cu" "B.Cu") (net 1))
 (segment (start 56.515 55.245) (end 55.325 54.055) (width 1) (layer "B.Cu") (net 1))
 (segment (start 68.58 60.96) (end 68.58 58.42) (width 1) (layer "B.Cu") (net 1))
 (segment (start 78.74 59.055) (end 74.295 59.055) (width 1) (layer "B.Cu") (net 1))
 (segment (start 55.325 54.055) (end 53.34 54.055) (width 1) (layer "B.Cu") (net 1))
 (segment (start 74.295 59.055) (end 73.66 58.42) (width 1) (layer "B.Cu") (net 1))
 (segment (start 63.5 60.96) (end 63.5 59.69) (width 1) (layer "B.Cu") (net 5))
 (segment (start 68.58 54.61) (end 68.58 49.784) (width 1) (layer "B.Cu") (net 5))
 (segment (start 63.5 59.69) (end 68.58 54.61) (width 1) (layer "B.Cu") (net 5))
 (segment (start 60.96 62.23) (end 62.23 63.5) (width 1) (layer "B.Cu") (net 6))
 (segment (start 63.58 49.465) (end 63.58 55.8) (width 1) (layer "B.Cu") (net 6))
 (segment (start 62.23 63.5) (end 63.5 63.5) (width 1) (layer "B.Cu") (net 6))
 (segment (start 63.58 55.8) (end 60.96 58.42) (width 1) (layer "B.Cu") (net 6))
 (segment (start 60.96 58.42) (end 60.96 62.23) (width 1) (layer "B.Cu") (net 6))
 (segment (start 59.69 54.61) (end 73.66 54.61) (width 1) (layer "F.Cu") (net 2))
 (via (at 59.69 54.61) (size 1.2) (drill 0.6) (layers "F.Cu" "B.Cu") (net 2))
 (via (at 73.66 54.61) (size 1.2) (drill 0.6) (layers "F.Cu" "B.Cu") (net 2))
 (segment (start 69.85 63.5) (end 68.58 63.5) (width 1) (layer "B.Cu") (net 2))
 (segment (start 74.215 54.055) (end 78.74 54.055) (width 1) (layer "B.Cu") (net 2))
 (segment (start 53.34 59.055) (end 56.515 59.055) (width 1) (layer "B.Cu") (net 2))
 (segment (start 73.66 54.61) (end 74.215 54.055) (width 1) (layer "B.Cu") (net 2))
 (segment (start 59.69 55.88) (end 59.69 54.61) (width 1) (layer "B.Cu") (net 2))
 (segment (start 73.66 54.61) (end 71.12 57.15) (width 1) (layer "B.Cu") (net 2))
 (segment (start 71.12 57.15) (end 71.12 62.23) (width 1) (layer "B.Cu") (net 2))
 (segment (start 71.12 62.23) (end 69.85 63.5) (width 1) (layer "B.Cu") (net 2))
 (segment (start 56.515 59.055) (end 59.69 55.88) (width 1) (layer "B.Cu") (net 2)))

